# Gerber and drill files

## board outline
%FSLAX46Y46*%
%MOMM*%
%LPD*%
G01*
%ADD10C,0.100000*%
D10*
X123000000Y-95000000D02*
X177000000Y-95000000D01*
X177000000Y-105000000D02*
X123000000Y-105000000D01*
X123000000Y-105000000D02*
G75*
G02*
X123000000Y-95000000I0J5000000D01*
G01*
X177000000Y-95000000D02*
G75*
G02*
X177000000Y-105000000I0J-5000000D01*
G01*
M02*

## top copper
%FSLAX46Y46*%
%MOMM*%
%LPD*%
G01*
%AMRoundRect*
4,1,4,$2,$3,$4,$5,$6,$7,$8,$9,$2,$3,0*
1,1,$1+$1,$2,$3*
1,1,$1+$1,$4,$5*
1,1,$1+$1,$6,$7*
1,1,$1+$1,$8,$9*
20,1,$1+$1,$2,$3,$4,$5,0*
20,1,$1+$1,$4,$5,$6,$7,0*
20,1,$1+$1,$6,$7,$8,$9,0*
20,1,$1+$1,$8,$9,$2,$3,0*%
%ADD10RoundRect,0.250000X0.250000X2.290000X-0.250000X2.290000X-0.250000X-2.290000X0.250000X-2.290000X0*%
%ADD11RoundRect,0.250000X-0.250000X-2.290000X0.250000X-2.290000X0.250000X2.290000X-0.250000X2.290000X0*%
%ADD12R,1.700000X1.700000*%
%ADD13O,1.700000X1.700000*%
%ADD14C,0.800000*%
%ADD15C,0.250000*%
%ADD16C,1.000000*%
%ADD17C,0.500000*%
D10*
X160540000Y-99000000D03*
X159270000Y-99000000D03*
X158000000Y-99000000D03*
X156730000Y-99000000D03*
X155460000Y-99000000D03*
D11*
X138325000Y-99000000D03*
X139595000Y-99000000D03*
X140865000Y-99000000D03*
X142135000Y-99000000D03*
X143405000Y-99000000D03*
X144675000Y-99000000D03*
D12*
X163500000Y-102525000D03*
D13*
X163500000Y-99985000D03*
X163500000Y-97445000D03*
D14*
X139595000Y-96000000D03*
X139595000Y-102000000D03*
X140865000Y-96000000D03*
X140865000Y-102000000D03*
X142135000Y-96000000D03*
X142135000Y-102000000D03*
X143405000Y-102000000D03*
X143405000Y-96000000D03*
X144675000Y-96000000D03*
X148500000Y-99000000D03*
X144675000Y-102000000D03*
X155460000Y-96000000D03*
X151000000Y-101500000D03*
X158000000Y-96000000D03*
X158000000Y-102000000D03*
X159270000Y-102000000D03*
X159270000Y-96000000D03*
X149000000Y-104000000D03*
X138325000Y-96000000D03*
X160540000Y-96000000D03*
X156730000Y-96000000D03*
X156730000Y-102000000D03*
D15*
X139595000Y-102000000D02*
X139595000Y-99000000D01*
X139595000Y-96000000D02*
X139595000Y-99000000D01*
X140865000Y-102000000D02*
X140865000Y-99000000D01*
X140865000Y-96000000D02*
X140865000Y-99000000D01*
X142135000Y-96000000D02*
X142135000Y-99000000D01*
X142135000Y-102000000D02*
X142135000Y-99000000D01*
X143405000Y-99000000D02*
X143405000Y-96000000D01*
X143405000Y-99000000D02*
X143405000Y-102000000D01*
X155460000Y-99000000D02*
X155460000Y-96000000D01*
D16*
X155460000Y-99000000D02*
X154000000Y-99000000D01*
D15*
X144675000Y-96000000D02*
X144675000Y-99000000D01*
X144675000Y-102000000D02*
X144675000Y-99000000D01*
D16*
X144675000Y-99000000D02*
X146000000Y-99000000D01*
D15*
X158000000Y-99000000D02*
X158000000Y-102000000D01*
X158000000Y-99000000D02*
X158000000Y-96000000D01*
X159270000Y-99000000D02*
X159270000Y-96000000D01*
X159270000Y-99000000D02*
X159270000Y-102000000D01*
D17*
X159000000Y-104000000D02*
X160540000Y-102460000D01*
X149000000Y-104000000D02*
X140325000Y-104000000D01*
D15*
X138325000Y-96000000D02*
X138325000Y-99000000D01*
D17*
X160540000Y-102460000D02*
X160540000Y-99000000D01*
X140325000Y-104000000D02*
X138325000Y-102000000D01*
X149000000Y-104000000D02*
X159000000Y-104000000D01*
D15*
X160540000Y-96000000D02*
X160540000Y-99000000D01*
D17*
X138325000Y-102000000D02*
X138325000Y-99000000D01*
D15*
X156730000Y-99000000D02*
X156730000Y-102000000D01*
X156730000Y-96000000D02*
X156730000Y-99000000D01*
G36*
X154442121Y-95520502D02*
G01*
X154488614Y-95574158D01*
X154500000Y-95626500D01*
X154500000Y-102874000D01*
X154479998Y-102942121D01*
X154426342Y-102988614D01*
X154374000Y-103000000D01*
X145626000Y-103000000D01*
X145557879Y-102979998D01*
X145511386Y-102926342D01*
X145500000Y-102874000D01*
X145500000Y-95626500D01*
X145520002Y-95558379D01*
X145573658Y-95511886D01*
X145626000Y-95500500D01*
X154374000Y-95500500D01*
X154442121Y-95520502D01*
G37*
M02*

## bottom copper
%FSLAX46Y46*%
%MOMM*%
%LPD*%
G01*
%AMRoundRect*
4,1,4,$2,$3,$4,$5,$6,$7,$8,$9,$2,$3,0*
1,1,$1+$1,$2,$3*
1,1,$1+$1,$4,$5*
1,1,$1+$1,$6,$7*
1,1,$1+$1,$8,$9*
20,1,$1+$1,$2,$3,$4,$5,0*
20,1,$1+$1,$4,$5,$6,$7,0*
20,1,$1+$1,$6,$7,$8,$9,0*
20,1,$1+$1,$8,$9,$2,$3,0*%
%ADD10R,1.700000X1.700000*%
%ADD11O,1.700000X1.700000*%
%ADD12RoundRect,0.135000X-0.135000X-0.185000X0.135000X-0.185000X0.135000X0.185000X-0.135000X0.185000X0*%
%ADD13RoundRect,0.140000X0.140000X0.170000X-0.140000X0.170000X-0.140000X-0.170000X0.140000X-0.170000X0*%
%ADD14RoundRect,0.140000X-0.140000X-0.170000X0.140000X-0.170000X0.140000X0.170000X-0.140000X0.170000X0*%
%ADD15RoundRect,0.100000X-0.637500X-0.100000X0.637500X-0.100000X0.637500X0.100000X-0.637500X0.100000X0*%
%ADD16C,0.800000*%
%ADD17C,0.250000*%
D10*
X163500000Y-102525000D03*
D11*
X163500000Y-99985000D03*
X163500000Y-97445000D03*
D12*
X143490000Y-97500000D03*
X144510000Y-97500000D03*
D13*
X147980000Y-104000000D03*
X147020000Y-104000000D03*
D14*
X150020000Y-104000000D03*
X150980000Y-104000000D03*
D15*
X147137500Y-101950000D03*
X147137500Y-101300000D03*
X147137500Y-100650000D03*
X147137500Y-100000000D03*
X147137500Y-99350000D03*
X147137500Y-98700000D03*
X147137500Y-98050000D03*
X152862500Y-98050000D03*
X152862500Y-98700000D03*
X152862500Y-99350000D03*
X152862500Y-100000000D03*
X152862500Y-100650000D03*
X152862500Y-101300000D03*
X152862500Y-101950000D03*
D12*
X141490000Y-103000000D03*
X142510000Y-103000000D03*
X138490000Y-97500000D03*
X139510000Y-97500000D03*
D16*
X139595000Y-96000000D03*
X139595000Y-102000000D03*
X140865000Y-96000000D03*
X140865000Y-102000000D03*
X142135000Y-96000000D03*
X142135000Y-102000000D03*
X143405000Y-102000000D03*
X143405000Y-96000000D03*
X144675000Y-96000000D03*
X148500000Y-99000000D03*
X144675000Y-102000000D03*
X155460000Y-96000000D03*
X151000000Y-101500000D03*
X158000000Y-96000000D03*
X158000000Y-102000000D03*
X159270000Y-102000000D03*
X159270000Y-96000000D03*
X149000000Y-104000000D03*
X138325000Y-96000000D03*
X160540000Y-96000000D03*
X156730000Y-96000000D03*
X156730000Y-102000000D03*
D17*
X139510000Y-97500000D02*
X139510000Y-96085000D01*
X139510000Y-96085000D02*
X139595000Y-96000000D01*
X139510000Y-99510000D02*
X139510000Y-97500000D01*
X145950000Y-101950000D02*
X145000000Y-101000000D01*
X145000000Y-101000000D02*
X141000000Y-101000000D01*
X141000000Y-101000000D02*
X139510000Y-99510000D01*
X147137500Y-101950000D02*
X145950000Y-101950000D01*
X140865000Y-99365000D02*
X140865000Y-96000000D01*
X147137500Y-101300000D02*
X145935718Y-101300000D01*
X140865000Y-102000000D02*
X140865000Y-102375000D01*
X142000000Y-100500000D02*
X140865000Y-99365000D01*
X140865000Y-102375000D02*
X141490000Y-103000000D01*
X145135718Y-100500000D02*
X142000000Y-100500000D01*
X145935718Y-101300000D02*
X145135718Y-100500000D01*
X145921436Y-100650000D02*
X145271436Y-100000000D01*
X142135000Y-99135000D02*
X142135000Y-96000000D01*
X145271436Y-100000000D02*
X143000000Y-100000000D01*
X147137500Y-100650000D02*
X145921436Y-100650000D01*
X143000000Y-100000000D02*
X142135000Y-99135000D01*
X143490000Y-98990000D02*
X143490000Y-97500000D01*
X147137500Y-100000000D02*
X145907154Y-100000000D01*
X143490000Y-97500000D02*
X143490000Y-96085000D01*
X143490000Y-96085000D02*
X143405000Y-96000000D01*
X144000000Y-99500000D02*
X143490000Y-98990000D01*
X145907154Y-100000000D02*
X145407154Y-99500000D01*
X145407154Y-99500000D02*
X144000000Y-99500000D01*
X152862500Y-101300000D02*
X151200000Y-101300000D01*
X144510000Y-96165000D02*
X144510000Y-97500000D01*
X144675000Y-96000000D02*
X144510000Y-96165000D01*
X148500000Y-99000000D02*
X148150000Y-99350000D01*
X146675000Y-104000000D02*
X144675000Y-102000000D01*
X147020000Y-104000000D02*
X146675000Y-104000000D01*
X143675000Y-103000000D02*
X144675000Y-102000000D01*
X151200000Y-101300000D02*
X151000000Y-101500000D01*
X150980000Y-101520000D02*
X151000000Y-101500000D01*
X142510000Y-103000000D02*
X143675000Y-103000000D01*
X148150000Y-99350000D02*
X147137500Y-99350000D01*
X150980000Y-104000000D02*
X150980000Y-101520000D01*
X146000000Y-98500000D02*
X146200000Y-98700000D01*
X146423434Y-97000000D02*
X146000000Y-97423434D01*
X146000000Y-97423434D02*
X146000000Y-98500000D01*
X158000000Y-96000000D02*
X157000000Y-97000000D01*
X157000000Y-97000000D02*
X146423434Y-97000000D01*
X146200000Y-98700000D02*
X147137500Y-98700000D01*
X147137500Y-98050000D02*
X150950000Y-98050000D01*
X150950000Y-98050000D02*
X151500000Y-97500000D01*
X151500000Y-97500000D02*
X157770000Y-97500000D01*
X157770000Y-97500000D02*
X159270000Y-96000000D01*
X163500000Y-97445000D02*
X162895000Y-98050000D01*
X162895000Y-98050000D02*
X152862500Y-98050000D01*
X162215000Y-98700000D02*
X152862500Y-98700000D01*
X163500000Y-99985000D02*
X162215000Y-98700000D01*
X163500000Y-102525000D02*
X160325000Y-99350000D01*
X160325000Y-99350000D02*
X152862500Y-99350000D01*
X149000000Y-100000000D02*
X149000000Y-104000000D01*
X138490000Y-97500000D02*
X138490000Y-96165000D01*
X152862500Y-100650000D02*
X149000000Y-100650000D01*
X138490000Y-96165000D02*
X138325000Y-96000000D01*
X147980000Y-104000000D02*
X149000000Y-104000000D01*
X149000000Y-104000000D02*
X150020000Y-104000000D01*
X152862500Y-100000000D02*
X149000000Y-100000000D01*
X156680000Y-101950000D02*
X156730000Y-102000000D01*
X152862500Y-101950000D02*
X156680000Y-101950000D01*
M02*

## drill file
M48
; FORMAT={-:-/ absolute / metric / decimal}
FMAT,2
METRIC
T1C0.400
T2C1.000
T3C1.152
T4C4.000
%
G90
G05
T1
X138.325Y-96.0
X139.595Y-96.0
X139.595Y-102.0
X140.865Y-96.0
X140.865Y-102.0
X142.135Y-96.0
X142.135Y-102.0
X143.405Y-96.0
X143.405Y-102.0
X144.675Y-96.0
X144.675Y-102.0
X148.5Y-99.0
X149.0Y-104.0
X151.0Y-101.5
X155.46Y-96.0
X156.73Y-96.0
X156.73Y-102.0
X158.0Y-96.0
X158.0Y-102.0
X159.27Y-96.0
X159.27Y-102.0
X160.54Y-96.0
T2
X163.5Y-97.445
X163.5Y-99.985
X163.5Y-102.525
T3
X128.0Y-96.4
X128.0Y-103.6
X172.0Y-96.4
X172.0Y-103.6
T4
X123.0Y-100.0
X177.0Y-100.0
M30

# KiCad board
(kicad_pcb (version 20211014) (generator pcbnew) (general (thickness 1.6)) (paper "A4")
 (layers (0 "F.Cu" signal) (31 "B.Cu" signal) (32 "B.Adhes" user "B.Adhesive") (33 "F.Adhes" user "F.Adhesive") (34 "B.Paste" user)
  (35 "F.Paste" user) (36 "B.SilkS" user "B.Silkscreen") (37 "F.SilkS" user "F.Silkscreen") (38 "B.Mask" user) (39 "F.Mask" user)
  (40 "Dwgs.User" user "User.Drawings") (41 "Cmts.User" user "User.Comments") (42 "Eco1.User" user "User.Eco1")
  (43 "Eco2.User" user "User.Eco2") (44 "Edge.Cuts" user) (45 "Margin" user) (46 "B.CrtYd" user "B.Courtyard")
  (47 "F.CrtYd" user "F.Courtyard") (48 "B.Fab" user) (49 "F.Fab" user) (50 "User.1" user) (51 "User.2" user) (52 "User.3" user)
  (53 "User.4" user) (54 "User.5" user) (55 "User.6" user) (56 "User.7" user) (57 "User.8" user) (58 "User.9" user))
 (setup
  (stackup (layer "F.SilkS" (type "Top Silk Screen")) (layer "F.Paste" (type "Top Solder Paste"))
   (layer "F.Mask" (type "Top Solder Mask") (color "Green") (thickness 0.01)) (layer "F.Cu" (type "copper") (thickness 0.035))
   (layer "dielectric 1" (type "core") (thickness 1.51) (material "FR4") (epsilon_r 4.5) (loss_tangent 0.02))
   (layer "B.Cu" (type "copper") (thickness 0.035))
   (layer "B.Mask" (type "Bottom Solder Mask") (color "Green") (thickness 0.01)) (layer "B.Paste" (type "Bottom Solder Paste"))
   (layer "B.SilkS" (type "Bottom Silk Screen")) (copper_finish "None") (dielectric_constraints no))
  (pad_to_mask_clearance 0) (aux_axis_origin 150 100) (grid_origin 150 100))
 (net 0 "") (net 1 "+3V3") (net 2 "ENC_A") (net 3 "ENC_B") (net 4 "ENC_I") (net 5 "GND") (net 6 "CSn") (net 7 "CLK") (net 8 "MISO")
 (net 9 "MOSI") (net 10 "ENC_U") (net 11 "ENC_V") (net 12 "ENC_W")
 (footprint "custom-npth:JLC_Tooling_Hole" (layer "F.Cu") (at 128 103.6)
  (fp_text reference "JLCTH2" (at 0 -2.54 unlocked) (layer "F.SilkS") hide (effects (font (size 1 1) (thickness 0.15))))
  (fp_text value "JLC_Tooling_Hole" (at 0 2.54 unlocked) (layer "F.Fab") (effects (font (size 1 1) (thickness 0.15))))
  (pad "" np_thru_hole circle (at 0 0) (size 1.3 1.3) (drill 1.152) (layers *.Mask) (solder_mask_margin 0.074) (clearance 0.248)
   (zone_connect 0)))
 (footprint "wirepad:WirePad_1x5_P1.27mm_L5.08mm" (layer "F.Cu") (at 158 99 180)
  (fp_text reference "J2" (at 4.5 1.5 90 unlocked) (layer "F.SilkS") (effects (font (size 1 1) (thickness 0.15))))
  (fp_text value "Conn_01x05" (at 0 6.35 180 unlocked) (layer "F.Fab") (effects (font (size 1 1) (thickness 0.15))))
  (pad "1" smd roundrect (at -2.54 0 180) (size 1 5.08) (layers "F.Cu" "F.Paste" "F.Mask") (roundrect_rratio 0.25) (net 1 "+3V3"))
  (pad "2" smd roundrect (at -1.27 0 180) (size 1 5.08) (layers "F.Cu" "F.Paste" "F.Mask") (roundrect_rratio 0.25) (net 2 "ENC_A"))
  (pad "3" smd roundrect (at 0 0 180) (size 1 5.08) (layers "F.Cu" "F.Paste" "F.Mask") (roundrect_rratio 0.25) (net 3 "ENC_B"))
  (pad "4" smd roundrect (at 1.27 0 180) (size 1 5.08) (layers "F.Cu" "F.Paste" "F.Mask") (roundrect_rratio 0.25) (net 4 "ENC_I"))
  (pad "5" smd roundrect (at 2.54 0 180) (size 1 5.08) (layers "F.Cu" "F.Paste" "F.Mask") (roundrect_rratio 0.25) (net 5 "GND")))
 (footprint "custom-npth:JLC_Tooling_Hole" (layer "F.Cu") (at 128 96.4)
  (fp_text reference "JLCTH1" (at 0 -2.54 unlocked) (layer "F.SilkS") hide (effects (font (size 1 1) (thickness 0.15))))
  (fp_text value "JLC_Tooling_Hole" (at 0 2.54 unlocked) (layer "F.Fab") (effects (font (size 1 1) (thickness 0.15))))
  (pad "" np_thru_hole circle (at 0 0) (size 1.3 1.3) (drill 1.152) (layers *.Mask) (solder_mask_margin 0.074) (clearance 0.248)
   (zone_connect 0)))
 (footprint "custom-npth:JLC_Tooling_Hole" (layer "F.Cu") (at 172 103.6)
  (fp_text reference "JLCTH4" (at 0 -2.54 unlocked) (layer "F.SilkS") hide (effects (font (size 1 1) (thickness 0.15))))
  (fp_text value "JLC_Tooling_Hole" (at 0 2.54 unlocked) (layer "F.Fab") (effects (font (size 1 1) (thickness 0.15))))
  (pad "" np_thru_hole circle (at 0 0) (size 1.3 1.3) (drill 1.152) (layers *.Mask) (solder_mask_margin 0.074) (clearance 0.248)
   (zone_connect 0)))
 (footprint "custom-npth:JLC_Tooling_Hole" (layer "F.Cu") (at 172 96.4)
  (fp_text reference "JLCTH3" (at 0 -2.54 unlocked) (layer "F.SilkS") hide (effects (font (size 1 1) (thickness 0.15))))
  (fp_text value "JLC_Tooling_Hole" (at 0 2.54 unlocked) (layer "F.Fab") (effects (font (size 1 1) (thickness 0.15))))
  (pad "" np_thru_hole circle (at 0 0) (size 1.3 1.3) (drill 1.152) (layers *.Mask) (solder_mask_margin 0.074) (clearance 0.248)
   (zone_connect 0)))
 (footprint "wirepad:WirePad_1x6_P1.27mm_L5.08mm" (layer "F.Cu") (at 141.5 99)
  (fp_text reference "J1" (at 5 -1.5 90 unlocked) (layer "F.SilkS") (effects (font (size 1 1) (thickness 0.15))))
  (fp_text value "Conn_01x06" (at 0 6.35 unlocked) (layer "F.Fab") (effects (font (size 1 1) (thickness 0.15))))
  (pad "1" smd roundrect (at -3.175 0) (size 1 5.08) (layers "F.Cu" "F.Paste" "F.Mask") (roundrect_rratio 0.25) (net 1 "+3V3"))
  (pad "2" smd roundrect (at -1.905 0) (size 1 5.08) (layers "F.Cu" "F.Paste" "F.Mask") (roundrect_rratio 0.25) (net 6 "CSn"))
  (pad "3" smd roundrect (at -0.635 0) (size 1 5.08) (layers "F.Cu" "F.Paste" "F.Mask") (roundrect_rratio 0.25) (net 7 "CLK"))
  (pad "4" smd roundrect (at 0.635 0) (size 1 5.08) (layers "F.Cu" "F.Paste" "F.Mask") (roundrect_rratio 0.25) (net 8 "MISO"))
  (pad "5" smd roundrect (at 1.905 0) (size 1 5.08) (layers "F.Cu" "F.Paste" "F.Mask") (roundrect_rratio 0.25) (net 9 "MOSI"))
  (pad "6" smd roundrect (at 3.175 0) (size 1 5.08) (layers "F.Cu" "F.Paste" "F.Mask") (roundrect_rratio 0.25) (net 5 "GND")))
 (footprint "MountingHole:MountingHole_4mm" (layer "F.Cu") (at 123 100)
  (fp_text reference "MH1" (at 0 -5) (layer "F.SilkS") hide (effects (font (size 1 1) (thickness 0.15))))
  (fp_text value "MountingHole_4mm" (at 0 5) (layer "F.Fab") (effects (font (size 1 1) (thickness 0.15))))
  (pad "" np_thru_hole circle (at 0 0) (size 4 4) (drill 4) (layers *.Cu *.Mask)))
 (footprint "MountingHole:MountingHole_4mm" (layer "F.Cu") (at 177 100)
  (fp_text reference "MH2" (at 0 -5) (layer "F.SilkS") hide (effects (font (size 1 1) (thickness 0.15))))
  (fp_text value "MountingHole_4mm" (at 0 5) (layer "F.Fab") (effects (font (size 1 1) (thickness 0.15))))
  (pad "" np_thru_hole circle (at 0 0) (size 4 4) (drill 4) (layers *.Cu *.Mask)))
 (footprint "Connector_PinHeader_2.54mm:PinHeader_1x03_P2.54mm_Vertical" (layer "F.Cu") (at 163.5 102.525 180)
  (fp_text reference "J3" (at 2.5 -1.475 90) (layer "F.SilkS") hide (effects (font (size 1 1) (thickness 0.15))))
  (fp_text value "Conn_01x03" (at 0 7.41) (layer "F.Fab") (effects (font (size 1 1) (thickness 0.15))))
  (pad "1" thru_hole rect (at 0 0 180) (size 1.7 1.7) (drill 1) (layers *.Cu *.Mask) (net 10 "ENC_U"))
  (pad "2" thru_hole oval (at 0 2.54 180) (size 1.7 1.7) (drill 1) (layers *.Cu *.Mask) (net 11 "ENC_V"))
  (pad "3" thru_hole oval (at 0 5.08 180) (size 1.7 1.7) (drill 1) (layers *.Cu *.Mask) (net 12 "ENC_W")))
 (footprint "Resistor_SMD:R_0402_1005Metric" (layer "B.Cu") (at 144 97.5)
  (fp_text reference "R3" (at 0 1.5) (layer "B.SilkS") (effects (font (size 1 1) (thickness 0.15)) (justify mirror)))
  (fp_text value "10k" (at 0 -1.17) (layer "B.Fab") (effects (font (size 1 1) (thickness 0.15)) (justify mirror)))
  (pad "1" smd roundrect (at -0.51 0) (size 0.54 0.64) (layers "B.Cu" "B.Paste" "B.Mask") (roundrect_rratio 0.25) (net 9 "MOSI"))
  (pad "2" smd roundrect (at 0.51 0) (size 0.54 0.64) (layers "B.Cu" "B.Paste" "B.Mask") (roundrect_rratio 0.25) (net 5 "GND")))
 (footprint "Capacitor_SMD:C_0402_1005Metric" (layer "B.Cu") (at 147.5 104 180)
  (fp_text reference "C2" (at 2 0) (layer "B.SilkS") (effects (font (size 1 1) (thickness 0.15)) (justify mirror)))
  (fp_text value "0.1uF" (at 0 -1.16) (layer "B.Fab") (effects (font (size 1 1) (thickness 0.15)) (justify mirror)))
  (pad "1" smd roundrect (at -0.48 0 180) (size 0.56 0.62) (layers "B.Cu" "B.Paste" "B.Mask") (roundrect_rratio 0.25) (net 1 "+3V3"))
  (pad "2" smd roundrect (at 0.48 0 180) (size 0.56 0.62) (layers "B.Cu" "B.Paste" "B.Mask") (roundrect_rratio 0.25) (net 5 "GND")))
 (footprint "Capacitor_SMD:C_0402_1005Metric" (layer "B.Cu") (at 150.5 104)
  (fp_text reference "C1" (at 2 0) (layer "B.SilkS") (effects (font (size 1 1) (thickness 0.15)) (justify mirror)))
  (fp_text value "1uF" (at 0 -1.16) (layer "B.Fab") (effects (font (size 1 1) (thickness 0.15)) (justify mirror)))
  (pad "1" smd roundrect (at -0.48 0) (size 0.56 0.62) (layers "B.Cu" "B.Paste" "B.Mask") (roundrect_rratio 0.25) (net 1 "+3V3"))
  (pad "2" smd roundrect (at 0.48 0) (size 0.56 0.62) (layers "B.Cu" "B.Paste" "B.Mask") (roundrect_rratio 0.25) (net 5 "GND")))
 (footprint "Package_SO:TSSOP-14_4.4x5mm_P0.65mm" (layer "B.Cu") (at 150 100)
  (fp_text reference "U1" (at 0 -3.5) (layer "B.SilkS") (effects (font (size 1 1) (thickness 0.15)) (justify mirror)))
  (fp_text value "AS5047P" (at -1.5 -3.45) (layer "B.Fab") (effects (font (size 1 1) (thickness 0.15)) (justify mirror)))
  (pad "1" smd roundrect (at -2.8625 1.95) (size 1.475 0.4) (layers "B.Cu" "B.Paste" "B.Mask") (roundrect_rratio 0.25) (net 6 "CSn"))
  (pad "2" smd roundrect (at -2.8625 1.3) (size 1.475 0.4) (layers "B.Cu" "B.Paste" "B.Mask") (roundrect_rratio 0.25) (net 7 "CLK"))
  (pad "3" smd roundrect (at -2.8625 0.65) (size 1.475 0.4) (layers "B.Cu" "B.Paste" "B.Mask") (roundrect_rratio 0.25) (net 8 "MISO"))
  (pad "4" smd roundrect (at -2.8625 0) (size 1.475 0.4) (layers "B.Cu" "B.Paste" "B.Mask") (roundrect_rratio 0.25) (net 9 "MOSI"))
  (pad "5" smd roundrect (at -2.8625 -0.65) (size 1.475 0.4) (layers "B.Cu" "B.Paste" "B.Mask") (roundrect_rratio 0.25) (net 5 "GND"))
  (pad "6" smd roundrect (at -2.8625 -1.3) (size 1.475 0.4) (layers "B.Cu" "B.Paste" "B.Mask") (roundrect_rratio 0.25) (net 3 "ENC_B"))
  (pad "7" smd roundrect (at -2.8625 -1.95) (size 1.475 0.4) (layers "B.Cu" "B.Paste" "B.Mask") (roundrect_rratio 0.25) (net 2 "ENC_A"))
  (pad "8" smd roundrect (at 2.8625 -1.95) (size 1.475 0.4) (layers "B.Cu" "B.Paste" "B.Mask") (roundrect_rratio 0.25) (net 12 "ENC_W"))
  (pad "9" smd roundrect (at 2.8625 -1.3) (size 1.475 0.4) (layers "B.Cu" "B.Paste" "B.Mask") (roundrect_rratio 0.25) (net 11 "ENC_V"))
  (pad "10" smd roundrect (at 2.8625 -0.65) (size 1.475 0.4) (layers "B.Cu" "B.Paste" "B.Mask") (roundrect_rratio 0.25) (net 10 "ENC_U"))
  (pad "11" smd roundrect (at 2.8625 0) (size 1.475 0.4) (layers "B.Cu" "B.Paste" "B.Mask") (roundrect_rratio 0.25) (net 1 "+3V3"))
  (pad "12" smd roundrect (at 2.8625 0.65) (size 1.475 0.4) (layers "B.Cu" "B.Paste" "B.Mask") (roundrect_rratio 0.25) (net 1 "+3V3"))
  (pad "13" smd roundrect (at 2.8625 1.3) (size 1.475 0.4) (layers "B.Cu" "B.Paste" "B.Mask") (roundrect_rratio 0.25) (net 5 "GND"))
  (pad "14" smd roundrect (at 2.8625 1.95) (size 1.475 0.4) (layers "B.Cu" "B.Paste" "B.Mask") (roundrect_rratio 0.25) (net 4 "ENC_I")))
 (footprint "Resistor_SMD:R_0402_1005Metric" (layer "B.Cu") (at 142 103)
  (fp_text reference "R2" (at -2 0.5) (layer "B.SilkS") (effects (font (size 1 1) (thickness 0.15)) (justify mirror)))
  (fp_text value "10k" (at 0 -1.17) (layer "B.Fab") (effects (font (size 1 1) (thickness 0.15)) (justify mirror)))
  (pad "1" smd roundrect (at -0.51 0) (size 0.54 0.64) (layers "B.Cu" "B.Paste" "B.Mask") (roundrect_rratio 0.25) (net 7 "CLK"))
  (pad "2" smd roundrect (at 0.51 0) (size 0.54 0.64) (layers "B.Cu" "B.Paste" "B.Mask") (roundrect_rratio 0.25) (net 5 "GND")))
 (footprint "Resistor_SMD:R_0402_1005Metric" (layer "B.Cu") (at 139 97.5)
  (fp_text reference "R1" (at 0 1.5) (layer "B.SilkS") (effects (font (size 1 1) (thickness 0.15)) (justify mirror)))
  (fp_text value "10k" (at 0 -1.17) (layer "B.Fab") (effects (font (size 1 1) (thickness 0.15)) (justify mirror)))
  (pad "1" smd roundrect (at -0.51 0) (size 0.54 0.64) (layers "B.Cu" "B.Paste" "B.Mask") (roundrect_rratio 0.25) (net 1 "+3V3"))
  (pad "2" smd roundrect (at 0.51 0) (size 0.54 0.64) (layers "B.Cu" "B.Paste" "B.Mask") (roundrect_rratio 0.25) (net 6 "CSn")))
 (gr_line (start 123 95) (end 177 95) (layer "Edge.Cuts") (width 0.1))
 (gr_line (start 177 105) (end 123 105) (layer "Edge.Cuts") (width 0.1))
 (gr_arc (start 123 105) (mid 118 100) (end 123 95) (layer "Edge.Cuts") (width 0.1))
 (gr_arc (start 177 95) (mid 182 100) (end 177 105) (layer "Edge.Cuts") (width 0.1))
 (segment (start 139.595 102) (end 139.595 99) (width 0.25) (layer "F.Cu") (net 6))
 (segment (start 139.595 96) (end 139.595 99) (width 0.25) (layer "F.Cu") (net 6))
 (via (at 139.595 96) (size 0.8) (drill 0.4) (layers "F.Cu" "B.Cu") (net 6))
 (via (at 139.595 102) (size 0.8) (drill 0.4) (layers "F.Cu" "B.Cu") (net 6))
 (segment (start 139.51 97.5) (end 139.51 96.085) (width 0.25) (layer "B.Cu") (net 6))
 (segment (start 139.51 96.085) (end 139.595 96) (width 0.25) (layer "B.Cu") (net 6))
 (segment (start 139.51 99.51) (end 139.51 97.5) (width 0.25) (layer "B.Cu") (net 6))
 (segment (start 145.95 101.95) (end 145 101) (width 0.25) (layer "B.Cu") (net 6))
 (segment (start 145 101) (end 141 101) (width 0.25) (layer "B.Cu") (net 6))
 (segment (start 141 101) (end 139.51 99.51) (width 0.25) (layer "B.Cu") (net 6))
 (segment (start 147.1375 101.95) (end 145.95 101.95) (width 0.25) (layer "B.Cu") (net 6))
 (segment (start 140.865 102) (end 140.865 99) (width 0.25) (layer "F.Cu") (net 7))
 (segment (start 140.865 96) (end 140.865 99) (width 0.25) (layer "F.Cu") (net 7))
 (via (at 140.865 96) (size 0.8) (drill 0.4) (layers "F.Cu" "B.Cu") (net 7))
 (via (at 140.865 102) (size 0.8) (drill 0.4) (layers "F.Cu" "B.Cu") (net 7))
 (segment (start 140.865 99.365) (end 140.865 96) (width 0.25) (layer "B.Cu") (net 7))
 (segment (start 147.1375 101.3) (end 145.935718 101.3) (width 0.25) (layer "B.Cu") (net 7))
 (segment (start 140.865 102) (end 140.865 102.375) (width 0.25) (layer "B.Cu") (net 7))
 (segment (start 142 100.5) (end 140.865 99.365) (width 0.25) (layer "B.Cu") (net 7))
 (segment (start 140.865 102.375) (end 141.49 103) (width 0.25) (layer "B.Cu") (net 7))
 (segment (start 145.135718 100.5) (end 142 100.5) (width 0.25) (layer "B.Cu") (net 7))
 (segment (start 145.935718 101.3) (end 145.135718 100.5) (width 0.25) (layer "B.Cu") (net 7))
 (segment (start 142.135 96) (end 142.135 99) (width 0.25) (layer "F.Cu") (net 8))
 (segment (start 142.135 102) (end 142.135 99) (width 0.25) (layer "F.Cu") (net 8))
 (via (at 142.135 96) (size 0.8) (drill 0.4) (layers "F.Cu" "B.Cu") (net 8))
 (via (at 142.135 102) (size 0.8) (drill 0.4) (layers "F.Cu" "B.Cu") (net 8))
 (segment (start 145.921436 100.65) (end 145.271436 100) (width 0.25) (layer "B.Cu") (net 8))
 (segment (start 142.135 99.135) (end 142.135 96) (width 0.25) (layer "B.Cu") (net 8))
 (segment (start 145.271436 100) (end 143 100) (width 0.25) (layer "B.Cu") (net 8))
 (segment (start 147.1375 100.65) (end 145.921436 100.65) (width 0.25) (layer "B.Cu") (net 8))
 (segment (start 143 100) (end 142.135 99.135) (width 0.25) (layer "B.Cu") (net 8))
 (segment (start 143.405 99) (end 143.405 96) (width 0.25) (layer "F.Cu") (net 9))
 (segment (start 143.405 99) (end 143.405 102) (width 0.25) (layer "F.Cu") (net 9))
 (via (at 143.405 102) (size 0.8) (drill 0.4) (layers "F.Cu" "B.Cu") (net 9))
 (via (at 143.405 96) (size 0.8) (drill 0.4) (layers "F.Cu" "B.Cu") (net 9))
 (segment (start 143.49 98.99) (end 143.49 97.5) (width 0.25) (layer "B.Cu") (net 9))
 (segment (start 147.1375 100) (end 145.907154 100) (width 0.25) (layer "B.Cu") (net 9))
 (segment (start 143.49 97.5) (end 143.49 96.085) (width 0.25) (layer "B.Cu") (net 9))
 (segment (start 143.49 96.085) (end 143.405 96) (width 0.25) (layer "B.Cu") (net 9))
 (segment (start 144 99.5) (end 143.49 98.99) (width 0.25) (layer "B.Cu") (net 9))
 (segment (start 145.907154 100) (end 145.407154 99.5) (width 0.25) (layer "B.Cu") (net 9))
 (segment (start 145.407154 99.5) (end 144 99.5) (width 0.25) (layer "B.Cu") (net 9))
 (segment (start 155.46 99) (end 155.46 96) (width 0.25) (layer "F.Cu") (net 5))
 (segment (start 155.46 99) (end 154 99) (width 1) (layer "F.Cu") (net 5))
 (segment (start 144.675 96) (end 144.675 99) (width 0.25) (layer "F.Cu") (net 5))
 (segment (start 144.675 102) (end 144.675 99) (width 0.25) (layer "F.Cu") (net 5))
 (segment (start 144.675 99) (end 146 99) (width 1) (layer "F.Cu") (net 5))
 (via (at 144.675 96) (size 0.8) (drill 0.4) (layers "F.Cu" "B.Cu") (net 5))
 (via (at 148.5 99) (size 0.8) (drill 0.4) (layers "F.Cu" "B.Cu") (free) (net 5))
 (via (at 144.675 102) (size 0.8) (drill 0.4) (layers "F.Cu" "B.Cu") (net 5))
 (via (at 155.46 96) (size 0.8) (drill 0.4) (layers "F.Cu" "B.Cu") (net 5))
 (via (at 151 101.5) (size 0.8) (drill 0.4) (layers "F.Cu" "B.Cu") (free) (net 5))
 (segment (start 152.8625 101.3) (end 151.2 101.3) (width 0.25) (layer "B.Cu") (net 5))
 (segment (start 144.51 96.165) (end 144.51 97.5) (width 0.25) (layer "B.Cu") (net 5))
 (segment (start 144.675 96) (end 144.51 96.165) (width 0.25) (layer "B.Cu") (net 5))
 (segment (start 148.5 99) (end 148.15 99.35) (width 0.25) (layer "B.Cu") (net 5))
 (segment (start 146.675 104) (end 144.675 102) (width 0.25) (layer "B.Cu") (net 5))
 (segment (start 147.02 104) (end 146.675 104) (width 0.25) (layer "B.Cu") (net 5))
 (segment (start 143.675 103) (end 144.675 102) (width 0.25) (layer "B.Cu") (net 5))
 (segment (start 151.2 101.3) (end 151 101.5) (width 0.25) (layer "B.Cu") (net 5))
 (segment (start 150.98 101.52) (end 151 101.5) (width 0.25) (layer "B.Cu") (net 5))
 (segment (start 142.51 103) (end 143.675 103) (width 0.25) (layer "B.Cu") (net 5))
 (segment (start 148.15 99.35) (end 147.1375 99.35) (width 0.25) (layer "B.Cu") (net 5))
 (segment (start 150.98 104) (end 150.98 101.52) (width 0.25) (layer "B.Cu") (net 5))
 (segment (start 158 99) (end 158 102) (width 0.25) (layer "F.Cu") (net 3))
 (segment (start 158 99) (end 158 96) (width 0.25) (layer "F.Cu") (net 3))
 (via (at 158 96) (size 0.8) (drill 0.4) (layers "F.Cu" "B.Cu") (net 3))
 (via (at 158 102) (size 0.8) (drill 0.4) (layers "F.Cu" "B.Cu") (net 3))
 (segment (start 146 98.5) (end 146.2 98.7) (width 0.25) (layer "B.Cu") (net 3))
 (segment (start 146.423434 97) (end 146 97.423434) (width 0.25) (layer "B.Cu") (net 3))
 (segment (start 146 97.423434) (end 146 98.5) (width 0.25) (layer "B.Cu") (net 3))
 (segment (start 158 96) (end 157 97) (width 0.25) (layer "B.Cu") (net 3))
 (segment (start 157 97) (end 146.423434 97) (width 0.25) (layer "B.Cu") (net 3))
 (segment (start 146.2 98.7) (end 147.1375 98.7) (width 0.25) (layer "B.Cu") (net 3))
 (segment (start 159.27 99) (end 159.27 96) (width 0.25) (layer "F.Cu") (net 2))
 (segment (start 159.27 99) (end 159.27 102) (width 0.25) (layer "F.Cu") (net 2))
 (via (at 159.27 102) (size 0.8) (drill 0.4) (layers "F.Cu" "B.Cu") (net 2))
 (via (at 159.27 96) (size 0.8) (drill 0.4) (layers "F.Cu" "B.Cu") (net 2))
 (segment (start 147.1375 98.05) (end 150.95 98.05) (width 0.25) (layer "B.Cu") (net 2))
 (segment (start 150.95 98.05) (end 151.5 97.5) (width 0.25) (layer "B.Cu") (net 2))
 (segment (start 151.5 97.5) (end 157.77 97.5) (width 0.25) (layer "B.Cu") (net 2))
 (segment (start 157.77 97.5) (end 159.27 96) (width 0.25) (layer "B.Cu") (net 2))
 (segment (start 163.5 97.445) (end 162.895 98.05) (width 0.25) (layer "B.Cu") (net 12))
 (segment (start 162.895 98.05) (end 152.8625 98.05) (width 0.25) (layer "B.Cu") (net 12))
 (segment (start 162.215 98.7) (end 152.8625 98.7) (width 0.25) (layer "B.Cu") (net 11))
 (segment (start 163.5 99.985) (end 162.215 98.7) (width 0.25) (layer "B.Cu") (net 11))
 (segment (start 163.5 102.525) (end 160.325 99.35) (width 0.25) (layer "B.Cu") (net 10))
 (segment (start 160.325 99.35) (end 152.8625 99.35) (width 0.25) (layer "B.Cu") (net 10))
 (segment (start 159 104) (end 160.54 102.46) (width 0.5) (layer "F.Cu") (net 1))
 (segment (start 149 104) (end 140.325 104) (width 0.5) (layer "F.Cu") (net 1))
 (segment (start 138.325 96) (end 138.325 99) (width 0.25) (layer "F.Cu") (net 1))
 (segment (start 160.54 102.46) (end 160.54 99) (width 0.5) (layer "F.Cu") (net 1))
 (segment (start 140.325 104) (end 138.325 102) (width 0.5) (layer "F.Cu") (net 1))
 (segment (start 149 104) (end 159 104) (width 0.5) (layer "F.Cu") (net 1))
 (segment (start 160.54 96) (end 160.54 99) (width 0.25) (layer "F.Cu") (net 1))
 (segment (start 138.325 102) (end 138.325 99) (width 0.5) (layer "F.Cu") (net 1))
 (via (at 149 104) (size 0.8) (drill 0.4) (layers "F.Cu" "B.Cu") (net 1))
 (via (at 138.325 96) (size 0.8) (drill 0.4) (layers "F.Cu" "B.Cu") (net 1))
 (via (at 160.54 96) (size 0.8) (drill 0.4) (layers "F.Cu" "B.Cu") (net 1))
 (segment (start 149 100) (end 149 104) (width 0.25) (layer "B.Cu") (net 1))
 (segment (start 138.49 97.5) (end 138.49 96.165) (width 0.25) (layer "B.Cu") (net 1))
 (segment (start 152.8625 100.65) (end 149 100.65) (width 0.25) (layer "B.Cu") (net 1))
 (segment (start 138.49 96.165) (end 138.325 96) (width 0.25) (layer "B.Cu") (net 1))
 (segment (start 147.98 104) (end 149 104) (width 0.25) (layer "B.Cu") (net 1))
 (segment (start 149 104) (end 150.02 104) (width 0.25) (layer "B.Cu") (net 1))
 (segment (start 152.8625 100) (end 149 100) (width 0.25) (layer "B.Cu") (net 1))
 (segment (start 156.73 99) (end 156.73 102) (width 0.25) (layer "F.Cu") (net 4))
 (segment (start 156.73 96) (end 156.73 99) (width 0.25) (layer "F.Cu") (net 4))
 (via (at 156.73 96) (size 0.8) (drill 0.4) (layers "F.Cu" "B.Cu") (free) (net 4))
 (via (at 156.73 102) (size 0.8) (drill 0.4) (layers "F.Cu" "B.Cu") (free) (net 4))
 (segment (start 156.68 101.95) (end 156.73 102) (width 0.25) (layer "B.Cu") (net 4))
 (segment (start 152.8625 101.95) (end 156.68 101.95) (width 0.25) (layer "B.Cu") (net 4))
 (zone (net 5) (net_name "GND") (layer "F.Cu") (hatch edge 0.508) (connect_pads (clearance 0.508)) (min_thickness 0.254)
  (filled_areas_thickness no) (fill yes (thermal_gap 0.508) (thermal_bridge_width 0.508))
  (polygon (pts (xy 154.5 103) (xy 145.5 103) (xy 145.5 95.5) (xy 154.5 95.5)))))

